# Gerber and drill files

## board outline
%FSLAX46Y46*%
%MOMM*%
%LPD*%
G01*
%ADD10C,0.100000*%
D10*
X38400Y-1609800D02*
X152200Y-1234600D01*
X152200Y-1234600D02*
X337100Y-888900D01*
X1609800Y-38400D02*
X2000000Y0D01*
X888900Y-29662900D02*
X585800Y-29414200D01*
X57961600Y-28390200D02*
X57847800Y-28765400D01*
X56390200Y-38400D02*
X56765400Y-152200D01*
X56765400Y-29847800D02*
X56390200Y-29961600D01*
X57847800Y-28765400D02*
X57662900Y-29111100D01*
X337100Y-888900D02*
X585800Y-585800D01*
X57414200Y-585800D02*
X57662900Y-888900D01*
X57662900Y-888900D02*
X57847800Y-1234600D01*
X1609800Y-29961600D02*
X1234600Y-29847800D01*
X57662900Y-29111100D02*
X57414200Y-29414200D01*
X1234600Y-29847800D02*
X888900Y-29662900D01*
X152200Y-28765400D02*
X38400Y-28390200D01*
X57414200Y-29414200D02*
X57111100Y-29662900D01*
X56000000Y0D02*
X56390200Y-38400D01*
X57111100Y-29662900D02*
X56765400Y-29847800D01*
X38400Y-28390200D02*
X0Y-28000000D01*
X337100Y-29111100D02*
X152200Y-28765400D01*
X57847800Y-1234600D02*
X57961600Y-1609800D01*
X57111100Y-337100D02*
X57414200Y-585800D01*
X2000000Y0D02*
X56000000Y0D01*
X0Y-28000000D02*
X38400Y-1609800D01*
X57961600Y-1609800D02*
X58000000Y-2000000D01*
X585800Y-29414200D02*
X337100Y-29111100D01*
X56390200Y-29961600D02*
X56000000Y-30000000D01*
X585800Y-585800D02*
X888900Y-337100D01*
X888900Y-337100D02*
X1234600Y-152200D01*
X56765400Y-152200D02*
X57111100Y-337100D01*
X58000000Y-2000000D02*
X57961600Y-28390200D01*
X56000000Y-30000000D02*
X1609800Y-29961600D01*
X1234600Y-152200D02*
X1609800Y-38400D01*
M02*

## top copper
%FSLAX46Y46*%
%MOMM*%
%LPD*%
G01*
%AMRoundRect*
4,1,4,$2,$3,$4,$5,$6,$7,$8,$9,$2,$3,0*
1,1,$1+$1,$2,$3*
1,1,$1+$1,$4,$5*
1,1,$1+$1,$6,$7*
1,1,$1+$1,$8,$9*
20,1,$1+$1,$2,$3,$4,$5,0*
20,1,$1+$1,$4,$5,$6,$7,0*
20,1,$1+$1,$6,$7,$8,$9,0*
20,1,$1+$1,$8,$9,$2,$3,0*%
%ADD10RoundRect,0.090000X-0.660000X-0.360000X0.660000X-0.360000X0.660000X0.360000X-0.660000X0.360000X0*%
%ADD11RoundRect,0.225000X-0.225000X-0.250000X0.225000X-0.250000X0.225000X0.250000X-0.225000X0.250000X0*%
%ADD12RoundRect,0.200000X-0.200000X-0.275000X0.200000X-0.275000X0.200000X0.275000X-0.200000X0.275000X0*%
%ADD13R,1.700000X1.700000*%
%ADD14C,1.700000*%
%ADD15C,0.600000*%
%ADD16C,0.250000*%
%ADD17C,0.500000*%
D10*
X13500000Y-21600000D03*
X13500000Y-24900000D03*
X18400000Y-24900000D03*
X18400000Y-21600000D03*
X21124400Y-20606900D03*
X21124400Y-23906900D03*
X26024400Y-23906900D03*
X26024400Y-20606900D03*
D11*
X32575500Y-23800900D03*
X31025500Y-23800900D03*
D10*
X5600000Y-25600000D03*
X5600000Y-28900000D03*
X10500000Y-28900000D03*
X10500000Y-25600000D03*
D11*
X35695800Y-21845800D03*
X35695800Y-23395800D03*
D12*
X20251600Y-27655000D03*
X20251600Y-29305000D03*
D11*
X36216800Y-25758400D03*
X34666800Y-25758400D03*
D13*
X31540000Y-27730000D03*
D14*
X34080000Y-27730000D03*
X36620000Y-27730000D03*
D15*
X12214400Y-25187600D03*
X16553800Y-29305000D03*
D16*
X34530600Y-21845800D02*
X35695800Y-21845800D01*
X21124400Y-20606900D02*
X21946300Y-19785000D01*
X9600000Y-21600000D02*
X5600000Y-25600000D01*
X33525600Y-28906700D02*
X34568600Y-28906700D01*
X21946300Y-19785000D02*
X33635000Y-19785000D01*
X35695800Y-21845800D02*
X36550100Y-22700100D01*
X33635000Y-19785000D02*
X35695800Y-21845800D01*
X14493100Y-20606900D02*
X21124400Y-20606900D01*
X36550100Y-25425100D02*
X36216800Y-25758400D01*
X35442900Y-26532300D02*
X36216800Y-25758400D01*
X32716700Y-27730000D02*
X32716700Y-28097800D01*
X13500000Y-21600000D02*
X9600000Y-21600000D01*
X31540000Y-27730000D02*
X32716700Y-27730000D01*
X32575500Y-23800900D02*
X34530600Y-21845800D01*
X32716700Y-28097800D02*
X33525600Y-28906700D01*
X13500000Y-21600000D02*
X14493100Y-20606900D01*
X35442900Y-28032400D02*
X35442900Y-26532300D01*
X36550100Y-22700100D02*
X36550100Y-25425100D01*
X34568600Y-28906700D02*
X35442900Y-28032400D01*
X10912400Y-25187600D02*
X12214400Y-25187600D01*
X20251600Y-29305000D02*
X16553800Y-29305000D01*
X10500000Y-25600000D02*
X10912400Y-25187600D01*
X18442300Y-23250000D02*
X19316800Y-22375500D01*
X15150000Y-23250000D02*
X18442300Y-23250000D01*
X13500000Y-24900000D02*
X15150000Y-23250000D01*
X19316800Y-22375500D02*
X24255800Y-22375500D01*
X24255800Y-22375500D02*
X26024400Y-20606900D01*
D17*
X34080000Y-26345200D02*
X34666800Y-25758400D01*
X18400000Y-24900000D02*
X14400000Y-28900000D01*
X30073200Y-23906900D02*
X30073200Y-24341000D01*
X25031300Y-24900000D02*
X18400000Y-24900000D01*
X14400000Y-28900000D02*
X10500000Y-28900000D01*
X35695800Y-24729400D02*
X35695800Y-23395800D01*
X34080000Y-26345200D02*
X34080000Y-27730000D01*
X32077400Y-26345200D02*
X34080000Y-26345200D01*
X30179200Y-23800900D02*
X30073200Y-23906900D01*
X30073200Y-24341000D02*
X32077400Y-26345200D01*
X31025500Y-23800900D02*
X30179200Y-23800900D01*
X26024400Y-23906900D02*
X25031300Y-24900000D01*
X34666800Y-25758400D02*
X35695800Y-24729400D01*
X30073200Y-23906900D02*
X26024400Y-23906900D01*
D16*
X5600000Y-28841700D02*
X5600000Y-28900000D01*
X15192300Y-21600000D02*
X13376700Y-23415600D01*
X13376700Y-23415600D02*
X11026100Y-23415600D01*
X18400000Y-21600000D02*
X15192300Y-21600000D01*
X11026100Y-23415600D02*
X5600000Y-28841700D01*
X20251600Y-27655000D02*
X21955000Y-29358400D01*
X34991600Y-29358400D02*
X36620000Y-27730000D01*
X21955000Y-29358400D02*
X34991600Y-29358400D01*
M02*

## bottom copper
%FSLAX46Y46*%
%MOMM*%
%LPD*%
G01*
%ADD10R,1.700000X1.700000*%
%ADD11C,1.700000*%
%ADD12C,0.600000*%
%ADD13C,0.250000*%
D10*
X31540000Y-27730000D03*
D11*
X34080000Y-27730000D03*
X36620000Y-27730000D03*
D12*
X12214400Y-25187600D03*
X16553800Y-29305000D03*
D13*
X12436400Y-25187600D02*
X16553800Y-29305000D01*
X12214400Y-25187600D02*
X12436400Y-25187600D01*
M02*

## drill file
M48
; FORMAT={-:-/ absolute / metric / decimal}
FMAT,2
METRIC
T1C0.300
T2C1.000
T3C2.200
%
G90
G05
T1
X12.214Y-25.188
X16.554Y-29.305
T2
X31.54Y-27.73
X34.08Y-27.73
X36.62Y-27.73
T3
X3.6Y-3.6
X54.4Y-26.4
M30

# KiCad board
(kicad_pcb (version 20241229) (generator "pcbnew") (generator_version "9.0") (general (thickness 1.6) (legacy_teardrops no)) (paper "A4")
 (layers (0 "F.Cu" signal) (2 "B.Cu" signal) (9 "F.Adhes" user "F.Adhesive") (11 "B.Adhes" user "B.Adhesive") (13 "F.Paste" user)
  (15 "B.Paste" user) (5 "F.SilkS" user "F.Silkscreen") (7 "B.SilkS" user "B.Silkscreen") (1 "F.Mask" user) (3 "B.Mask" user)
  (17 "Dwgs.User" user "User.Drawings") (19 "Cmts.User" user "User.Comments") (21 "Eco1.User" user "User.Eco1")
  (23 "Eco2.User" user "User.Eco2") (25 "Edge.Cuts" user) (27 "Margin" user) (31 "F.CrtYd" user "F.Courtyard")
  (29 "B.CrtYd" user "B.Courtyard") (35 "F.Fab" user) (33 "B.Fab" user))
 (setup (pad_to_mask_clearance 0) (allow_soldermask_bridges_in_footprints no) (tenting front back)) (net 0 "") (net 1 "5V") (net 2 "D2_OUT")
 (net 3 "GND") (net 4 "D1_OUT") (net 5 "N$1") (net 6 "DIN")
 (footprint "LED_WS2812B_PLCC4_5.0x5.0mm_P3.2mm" (layer "F.Cu") (at 15.95 23.25)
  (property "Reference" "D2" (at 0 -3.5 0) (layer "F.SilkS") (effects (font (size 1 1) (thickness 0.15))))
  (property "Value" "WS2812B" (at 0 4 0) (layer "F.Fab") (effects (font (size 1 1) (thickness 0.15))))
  (pad "1" smd roundrect (at -2.45 -1.65) (size 1.5 0.9) (layers "F.Cu" "F.Mask" "F.Paste") (roundrect_rratio 0.1) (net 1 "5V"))
  (pad "2" smd roundrect (at -2.45 1.65) (size 1.5 0.9) (layers "F.Cu" "F.Mask" "F.Paste") (roundrect_rratio 0.1) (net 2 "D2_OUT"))
  (pad "3" smd roundrect (at 2.45 1.65) (size 1.5 0.9) (layers "F.Cu" "F.Mask" "F.Paste") (roundrect_rratio 0.1) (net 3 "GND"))
  (pad "4" smd roundrect (at 2.45 -1.65) (size 1.5 0.9) (layers "F.Cu" "F.Mask" "F.Paste") (roundrect_rratio 0.1) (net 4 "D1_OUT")))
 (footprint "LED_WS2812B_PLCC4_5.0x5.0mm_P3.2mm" (layer "F.Cu") (at 23.5744 22.2569)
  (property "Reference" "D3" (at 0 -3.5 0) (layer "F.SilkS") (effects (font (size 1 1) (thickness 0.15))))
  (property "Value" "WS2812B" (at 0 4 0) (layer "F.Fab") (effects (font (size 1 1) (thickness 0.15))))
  (pad "1" smd roundrect (at -2.45 -1.65) (size 1.5 0.9) (layers "F.Cu" "F.Mask" "F.Paste") (roundrect_rratio 0.1) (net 1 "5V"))
  (pad "2" smd roundrect (at -2.45 1.65) (size 1.5 0.9) (layers "F.Cu" "F.Mask" "F.Paste") (roundrect_rratio 0.1))
  (pad "3" smd roundrect (at 2.45 1.65) (size 1.5 0.9) (layers "F.Cu" "F.Mask" "F.Paste") (roundrect_rratio 0.1) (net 3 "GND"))
  (pad "4" smd roundrect (at 2.45 -1.65) (size 1.5 0.9) (layers "F.Cu" "F.Mask" "F.Paste") (roundrect_rratio 0.1) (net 2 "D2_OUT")))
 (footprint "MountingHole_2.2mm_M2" (layer "F.Cu") (at 3.6 3.6)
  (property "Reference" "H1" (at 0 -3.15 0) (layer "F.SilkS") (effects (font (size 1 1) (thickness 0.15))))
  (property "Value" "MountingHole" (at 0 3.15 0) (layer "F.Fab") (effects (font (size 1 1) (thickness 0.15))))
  (pad "" np_thru_hole circle (at 0 0) (size 2.2 2.2) (drill 2.2) (layers "*.Cu" "*.Mask")))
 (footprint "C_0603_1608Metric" (layer "F.Cu") (at 31.8005 23.8009 180)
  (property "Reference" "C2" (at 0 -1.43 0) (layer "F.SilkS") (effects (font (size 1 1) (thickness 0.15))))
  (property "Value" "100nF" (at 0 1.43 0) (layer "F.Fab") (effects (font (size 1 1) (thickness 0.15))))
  (pad "1" smd roundrect (at -0.775 0) (size 0.9 0.95) (layers "F.Cu" "F.Mask" "F.Paste") (roundrect_rratio 0.25) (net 1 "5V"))
  (pad "2" smd roundrect (at 0.775 0) (size 0.9 0.95) (layers "F.Cu" "F.Mask" "F.Paste") (roundrect_rratio 0.25) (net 3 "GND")))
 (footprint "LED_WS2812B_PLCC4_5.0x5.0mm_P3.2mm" (layer "F.Cu") (at 8.05 27.25)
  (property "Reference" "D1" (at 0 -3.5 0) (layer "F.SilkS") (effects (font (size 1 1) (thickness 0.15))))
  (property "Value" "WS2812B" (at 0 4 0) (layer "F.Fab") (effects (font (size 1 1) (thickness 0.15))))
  (pad "1" smd roundrect (at -2.45 -1.65) (size 1.5 0.9) (layers "F.Cu" "F.Mask" "F.Paste") (roundrect_rratio 0.1) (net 1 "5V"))
  (pad "2" smd roundrect (at -2.45 1.65) (size 1.5 0.9) (layers "F.Cu" "F.Mask" "F.Paste") (roundrect_rratio 0.1) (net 4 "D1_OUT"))
  (pad "3" smd roundrect (at 2.45 1.65) (size 1.5 0.9) (layers "F.Cu" "F.Mask" "F.Paste") (roundrect_rratio 0.1) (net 3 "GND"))
  (pad "4" smd roundrect (at 2.45 -1.65) (size 1.5 0.9) (layers "F.Cu" "F.Mask" "F.Paste") (roundrect_rratio 0.1) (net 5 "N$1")))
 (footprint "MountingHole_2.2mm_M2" (layer "F.Cu") (at 54.4 26.4)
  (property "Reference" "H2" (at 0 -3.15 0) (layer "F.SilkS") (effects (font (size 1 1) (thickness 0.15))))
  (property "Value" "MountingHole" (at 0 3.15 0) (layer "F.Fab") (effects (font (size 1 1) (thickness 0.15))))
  (pad "" np_thru_hole circle (at 0 0) (size 2.2 2.2) (drill 2.2) (layers "*.Cu" "*.Mask")))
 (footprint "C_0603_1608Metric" (layer "F.Cu") (at 35.6958 22.6208 -90)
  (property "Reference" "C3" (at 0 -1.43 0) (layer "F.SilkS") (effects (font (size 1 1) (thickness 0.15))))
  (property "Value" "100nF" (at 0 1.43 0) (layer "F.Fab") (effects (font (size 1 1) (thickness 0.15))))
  (pad "1" smd roundrect (at -0.775 0) (size 0.9 0.95) (layers "F.Cu" "F.Mask" "F.Paste") (roundrect_rratio 0.25) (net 1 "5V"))
  (pad "2" smd roundrect (at 0.775 0) (size 0.9 0.95) (layers "F.Cu" "F.Mask" "F.Paste") (roundrect_rratio 0.25) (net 3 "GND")))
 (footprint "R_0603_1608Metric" (layer "F.Cu") (at 20.2516 28.48 -90)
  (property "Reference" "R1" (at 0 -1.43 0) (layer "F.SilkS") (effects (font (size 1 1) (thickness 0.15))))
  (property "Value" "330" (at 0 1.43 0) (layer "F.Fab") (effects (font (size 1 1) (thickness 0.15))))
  (pad "1" smd roundrect (at -0.825 0) (size 0.8 0.95) (layers "F.Cu" "F.Mask" "F.Paste") (roundrect_rratio 0.25) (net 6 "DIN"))
  (pad "2" smd roundrect (at 0.825 0) (size 0.8 0.95) (layers "F.Cu" "F.Mask" "F.Paste") (roundrect_rratio 0.25) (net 5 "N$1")))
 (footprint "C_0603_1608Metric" (layer "F.Cu") (at 35.4418 25.7584 180)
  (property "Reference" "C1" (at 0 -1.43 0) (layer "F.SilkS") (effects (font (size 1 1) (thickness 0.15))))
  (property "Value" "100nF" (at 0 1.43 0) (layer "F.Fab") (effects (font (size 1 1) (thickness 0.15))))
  (pad "1" smd roundrect (at -0.775 0) (size 0.9 0.95) (layers "F.Cu" "F.Mask" "F.Paste") (roundrect_rratio 0.25) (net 1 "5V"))
  (pad "2" smd roundrect (at 0.775 0) (size 0.9 0.95) (layers "F.Cu" "F.Mask" "F.Paste") (roundrect_rratio 0.25) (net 3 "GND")))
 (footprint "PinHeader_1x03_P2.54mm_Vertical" (layer "F.Cu") (at 31.54 27.73 90)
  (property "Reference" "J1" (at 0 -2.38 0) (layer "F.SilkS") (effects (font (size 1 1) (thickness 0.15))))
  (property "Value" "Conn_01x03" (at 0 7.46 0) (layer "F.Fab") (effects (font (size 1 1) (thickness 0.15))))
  (pad "1" thru_hole rect (at 0 0) (size 1.7 1.7) (drill 1) (layers "*.Cu" "*.Mask") (remove_unused_layers no) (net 1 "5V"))
  (pad "2" thru_hole circle (at 0 2.54) (size 1.7 1.7) (drill 1) (layers "*.Cu" "*.Mask") (remove_unused_layers no) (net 3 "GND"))
  (pad "3" thru_hole circle (at 0 5.08) (size 1.7 1.7) (drill 1) (layers "*.Cu" "*.Mask") (remove_unused_layers no) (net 6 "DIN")))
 (gr_line (start 0.0384 1.6098) (end 0.1522 1.2346) (stroke (width 0.1) (type solid)) (layer "Edge.Cuts"))
 (gr_line (start 0.1522 1.2346) (end 0.3371 0.8889) (stroke (width 0.1) (type solid)) (layer "Edge.Cuts"))
 (gr_line (start 1.6098 0.0384) (end 2 0) (stroke (width 0.1) (type solid)) (layer "Edge.Cuts"))
 (gr_line (start 0.8889 29.6629) (end 0.5858 29.4142) (stroke (width 0.1) (type solid)) (layer "Edge.Cuts"))
 (gr_line (start 57.9616 28.3902) (end 57.8478 28.7654) (stroke (width 0.1) (type solid)) (layer "Edge.Cuts"))
 (gr_line (start 56.3902 0.0384) (end 56.7654 0.1522) (stroke (width 0.1) (type solid)) (layer "Edge.Cuts"))
 (gr_line (start 56.7654 29.8478) (end 56.3902 29.9616) (stroke (width 0.1) (type solid)) (layer "Edge.Cuts"))
 (gr_line (start 57.8478 28.7654) (end 57.6629 29.1111) (stroke (width 0.1) (type solid)) (layer "Edge.Cuts"))
 (gr_line (start 0.3371 0.8889) (end 0.5858 0.5858) (stroke (width 0.1) (type solid)) (layer "Edge.Cuts"))
 (gr_line (start 57.4142 0.5858) (end 57.6629 0.8889) (stroke (width 0.1) (type solid)) (layer "Edge.Cuts"))
 (gr_line (start 57.6629 0.8889) (end 57.8478 1.2346) (stroke (width 0.1) (type solid)) (layer "Edge.Cuts"))
 (gr_line (start 1.6098 29.9616) (end 1.2346 29.8478) (stroke (width 0.1) (type solid)) (layer "Edge.Cuts"))
 (gr_line (start 57.6629 29.1111) (end 57.4142 29.4142) (stroke (width 0.1) (type solid)) (layer "Edge.Cuts"))
 (gr_line (start 1.2346 29.8478) (end 0.8889 29.6629) (stroke (width 0.1) (type solid)) (layer "Edge.Cuts"))
 (gr_line (start 0.1522 28.7654) (end 0.0384 28.3902) (stroke (width 0.1) (type solid)) (layer "Edge.Cuts"))
 (gr_line (start 57.4142 29.4142) (end 57.1111 29.6629) (stroke (width 0.1) (type solid)) (layer "Edge.Cuts"))
 (gr_line (start 56 0) (end 56.3902 0.0384) (stroke (width 0.1) (type solid)) (layer "Edge.Cuts"))
 (gr_line (start 57.1111 29.6629) (end 56.7654 29.8478) (stroke (width 0.1) (type solid)) (layer "Edge.Cuts"))
 (gr_line (start 0.0384 28.3902) (end 0 28) (stroke (width 0.1) (type solid)) (layer "Edge.Cuts"))
 (gr_line (start 0.3371 29.1111) (end 0.1522 28.7654) (stroke (width 0.1) (type solid)) (layer "Edge.Cuts"))
 (gr_line (start 57.8478 1.2346) (end 57.9616 1.6098) (stroke (width 0.1) (type solid)) (layer "Edge.Cuts"))
 (gr_line (start 57.1111 0.3371) (end 57.4142 0.5858) (stroke (width 0.1) (type solid)) (layer "Edge.Cuts"))
 (gr_line (start 2 0) (end 56 0) (stroke (width 0.1) (type solid)) (layer "Edge.Cuts"))
 (gr_line (start 0 28) (end 0.0384 1.6098) (stroke (width 0.1) (type solid)) (layer "Edge.Cuts"))
 (gr_line (start 57.9616 1.6098) (end 58 2) (stroke (width 0.1) (type solid)) (layer "Edge.Cuts"))
 (gr_line (start 0.5858 29.4142) (end 0.3371 29.1111) (stroke (width 0.1) (type solid)) (layer "Edge.Cuts"))
 (gr_line (start 56.3902 29.9616) (end 56 30) (stroke (width 0.1) (type solid)) (layer "Edge.Cuts"))
 (gr_line (start 0.5858 0.5858) (end 0.8889 0.3371) (stroke (width 0.1) (type solid)) (layer "Edge.Cuts"))
 (gr_line (start 0.8889 0.3371) (end 1.2346 0.1522) (stroke (width 0.1) (type solid)) (layer "Edge.Cuts"))
 (gr_line (start 56.7654 0.1522) (end 57.1111 0.3371) (stroke (width 0.1) (type solid)) (layer "Edge.Cuts"))
 (gr_line (start 58 2) (end 57.9616 28.3902) (stroke (width 0.1) (type solid)) (layer "Edge.Cuts"))
 (gr_line (start 56 30) (end 1.6098 29.9616) (stroke (width 0.1) (type solid)) (layer "Edge.Cuts"))
 (gr_line (start 1.2346 0.1522) (end 1.6098 0.0384) (stroke (width 0.1) (type solid)) (layer "Edge.Cuts"))
 (segment (start 34.5306 21.8458) (end 35.6958 21.8458) (width 0.25) (layer "F.Cu") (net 1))
 (segment (start 21.1244 20.6069) (end 21.9463 19.785) (width 0.25) (layer "F.Cu") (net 1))
 (segment (start 9.6 21.6) (end 5.6 25.6) (width 0.25) (layer "F.Cu") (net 1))
 (segment (start 33.5256 28.9067) (end 34.5686 28.9067) (width 0.25) (layer "F.Cu") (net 1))
 (segment (start 21.9463 19.785) (end 33.635 19.785) (width 0.25) (layer "F.Cu") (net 1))
 (segment (start 35.6958 21.8458) (end 36.5501 22.7001) (width 0.25) (layer "F.Cu") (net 1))
 (segment (start 33.635 19.785) (end 35.6958 21.8458) (width 0.25) (layer "F.Cu") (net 1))
 (segment (start 14.4931 20.6069) (end 21.1244 20.6069) (width 0.25) (layer "F.Cu") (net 1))
 (segment (start 36.5501 25.4251) (end 36.2168 25.7584) (width 0.25) (layer "F.Cu") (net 1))
 (segment (start 35.4429 26.5323) (end 36.2168 25.7584) (width 0.25) (layer "F.Cu") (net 1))
 (segment (start 32.7167 27.73) (end 32.7167 28.0978) (width 0.25) (layer "F.Cu") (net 1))
 (segment (start 13.5 21.6) (end 9.6 21.6) (width 0.25) (layer "F.Cu") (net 1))
 (segment (start 31.54 27.73) (end 32.7167 27.73) (width 0.25) (layer "F.Cu") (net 1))
 (segment (start 32.5755 23.8009) (end 34.5306 21.8458) (width 0.25) (layer "F.Cu") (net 1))
 (segment (start 32.7167 28.0978) (end 33.5256 28.9067) (width 0.25) (layer "F.Cu") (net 1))
 (segment (start 13.5 21.6) (end 14.4931 20.6069) (width 0.25) (layer "F.Cu") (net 1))
 (segment (start 35.4429 28.0324) (end 35.4429 26.5323) (width 0.25) (layer "F.Cu") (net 1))
 (segment (start 36.5501 22.7001) (end 36.5501 25.4251) (width 0.25) (layer "F.Cu") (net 1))
 (segment (start 34.5686 28.9067) (end 35.4429 28.0324) (width 0.25) (layer "F.Cu") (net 1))
 (segment (start 10.9124 25.1876) (end 12.2144 25.1876) (width 0.25) (layer "F.Cu") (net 5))
 (segment (start 20.2516 29.305) (end 16.5538 29.305) (width 0.25) (layer "F.Cu") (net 5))
 (segment (start 10.5 25.6) (end 10.9124 25.1876) (width 0.25) (layer "F.Cu") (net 5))
 (via (at 12.2144 25.1876) (size 0.6) (drill 0.3) (layers "F.Cu" "B.Cu") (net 5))
 (via (at 16.5538 29.305) (size 0.6) (drill 0.3) (layers "F.Cu" "B.Cu") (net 5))
 (segment (start 12.4364 25.1876) (end 16.5538 29.305) (width 0.25) (layer "B.Cu") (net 5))
 (segment (start 12.2144 25.1876) (end 12.4364 25.1876) (width 0.25) (layer "B.Cu") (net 5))
 (segment (start 18.4423 23.25) (end 19.3168 22.3755) (width 0.25) (layer "F.Cu") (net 2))
 (segment (start 15.15 23.25) (end 18.4423 23.25) (width 0.25) (layer "F.Cu") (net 2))
 (segment (start 13.5 24.9) (end 15.15 23.25) (width 0.25) (layer "F.Cu") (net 2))
 (segment (start 19.3168 22.3755) (end 24.2558 22.3755) (width 0.25) (layer "F.Cu") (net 2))
 (segment (start 24.2558 22.3755) (end 26.0244 20.6069) (width 0.25) (layer "F.Cu") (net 2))
 (segment (start 34.08 26.3452) (end 34.6668 25.7584) (width 0.5) (layer "F.Cu") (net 3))
 (segment (start 18.4 24.9) (end 14.4 28.9) (width 0.5) (layer "F.Cu") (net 3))
 (segment (start 30.0732 23.9069) (end 30.0732 24.341) (width 0.5) (layer "F.Cu") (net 3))
 (segment (start 25.0313 24.9) (end 18.4 24.9) (width 0.5) (layer "F.Cu") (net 3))
 (segment (start 14.4 28.9) (end 10.5 28.9) (width 0.5) (layer "F.Cu") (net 3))
 (segment (start 35.6958 24.7294) (end 35.6958 23.3958) (width 0.5) (layer "F.Cu") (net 3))
 (segment (start 34.08 26.3452) (end 34.08 27.73) (width 0.5) (layer "F.Cu") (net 3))
 (segment (start 32.0774 26.3452) (end 34.08 26.3452) (width 0.5) (layer "F.Cu") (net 3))
 (segment (start 30.1792 23.8009) (end 30.0732 23.9069) (width 0.5) (layer "F.Cu") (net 3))
 (segment (start 30.0732 24.341) (end 32.0774 26.3452) (width 0.5) (layer "F.Cu") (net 3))
 (segment (start 31.0255 23.8009) (end 30.1792 23.8009) (width 0.5) (layer "F.Cu") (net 3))
 (segment (start 26.0244 23.9069) (end 25.0313 24.9) (width 0.5) (layer "F.Cu") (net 3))
 (segment (start 34.6668 25.7584) (end 35.6958 24.7294) (width 0.5) (layer "F.Cu") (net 3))
 (segment (start 30.0732 23.9069) (end 26.0244 23.9069) (width 0.5) (layer "F.Cu") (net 3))
 (segment (start 5.6 28.8417) (end 5.6 28.9) (width 0.25) (layer "F.Cu") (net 4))
 (segment (start 15.1923 21.6) (end 13.3767 23.4156) (width 0.25) (layer "F.Cu") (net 4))
 (segment (start 13.3767 23.4156) (end 11.0261 23.4156) (width 0.25) (layer "F.Cu") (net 4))
 (segment (start 18.4 21.6) (end 15.1923 21.6) (width 0.25) (layer "F.Cu") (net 4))
 (segment (start 11.0261 23.4156) (end 5.6 28.8417) (width 0.25) (layer "F.Cu") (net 4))
 (segment (start 20.2516 27.655) (end 21.955 29.3584) (width 0.25) (layer "F.Cu") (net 6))
 (segment (start 34.9916 29.3584) (end 36.62 27.73) (width 0.25) (layer "F.Cu") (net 6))
 (segment (start 21.955 29.3584) (end 34.9916 29.3584) (width 0.25) (layer "F.Cu") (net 6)))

